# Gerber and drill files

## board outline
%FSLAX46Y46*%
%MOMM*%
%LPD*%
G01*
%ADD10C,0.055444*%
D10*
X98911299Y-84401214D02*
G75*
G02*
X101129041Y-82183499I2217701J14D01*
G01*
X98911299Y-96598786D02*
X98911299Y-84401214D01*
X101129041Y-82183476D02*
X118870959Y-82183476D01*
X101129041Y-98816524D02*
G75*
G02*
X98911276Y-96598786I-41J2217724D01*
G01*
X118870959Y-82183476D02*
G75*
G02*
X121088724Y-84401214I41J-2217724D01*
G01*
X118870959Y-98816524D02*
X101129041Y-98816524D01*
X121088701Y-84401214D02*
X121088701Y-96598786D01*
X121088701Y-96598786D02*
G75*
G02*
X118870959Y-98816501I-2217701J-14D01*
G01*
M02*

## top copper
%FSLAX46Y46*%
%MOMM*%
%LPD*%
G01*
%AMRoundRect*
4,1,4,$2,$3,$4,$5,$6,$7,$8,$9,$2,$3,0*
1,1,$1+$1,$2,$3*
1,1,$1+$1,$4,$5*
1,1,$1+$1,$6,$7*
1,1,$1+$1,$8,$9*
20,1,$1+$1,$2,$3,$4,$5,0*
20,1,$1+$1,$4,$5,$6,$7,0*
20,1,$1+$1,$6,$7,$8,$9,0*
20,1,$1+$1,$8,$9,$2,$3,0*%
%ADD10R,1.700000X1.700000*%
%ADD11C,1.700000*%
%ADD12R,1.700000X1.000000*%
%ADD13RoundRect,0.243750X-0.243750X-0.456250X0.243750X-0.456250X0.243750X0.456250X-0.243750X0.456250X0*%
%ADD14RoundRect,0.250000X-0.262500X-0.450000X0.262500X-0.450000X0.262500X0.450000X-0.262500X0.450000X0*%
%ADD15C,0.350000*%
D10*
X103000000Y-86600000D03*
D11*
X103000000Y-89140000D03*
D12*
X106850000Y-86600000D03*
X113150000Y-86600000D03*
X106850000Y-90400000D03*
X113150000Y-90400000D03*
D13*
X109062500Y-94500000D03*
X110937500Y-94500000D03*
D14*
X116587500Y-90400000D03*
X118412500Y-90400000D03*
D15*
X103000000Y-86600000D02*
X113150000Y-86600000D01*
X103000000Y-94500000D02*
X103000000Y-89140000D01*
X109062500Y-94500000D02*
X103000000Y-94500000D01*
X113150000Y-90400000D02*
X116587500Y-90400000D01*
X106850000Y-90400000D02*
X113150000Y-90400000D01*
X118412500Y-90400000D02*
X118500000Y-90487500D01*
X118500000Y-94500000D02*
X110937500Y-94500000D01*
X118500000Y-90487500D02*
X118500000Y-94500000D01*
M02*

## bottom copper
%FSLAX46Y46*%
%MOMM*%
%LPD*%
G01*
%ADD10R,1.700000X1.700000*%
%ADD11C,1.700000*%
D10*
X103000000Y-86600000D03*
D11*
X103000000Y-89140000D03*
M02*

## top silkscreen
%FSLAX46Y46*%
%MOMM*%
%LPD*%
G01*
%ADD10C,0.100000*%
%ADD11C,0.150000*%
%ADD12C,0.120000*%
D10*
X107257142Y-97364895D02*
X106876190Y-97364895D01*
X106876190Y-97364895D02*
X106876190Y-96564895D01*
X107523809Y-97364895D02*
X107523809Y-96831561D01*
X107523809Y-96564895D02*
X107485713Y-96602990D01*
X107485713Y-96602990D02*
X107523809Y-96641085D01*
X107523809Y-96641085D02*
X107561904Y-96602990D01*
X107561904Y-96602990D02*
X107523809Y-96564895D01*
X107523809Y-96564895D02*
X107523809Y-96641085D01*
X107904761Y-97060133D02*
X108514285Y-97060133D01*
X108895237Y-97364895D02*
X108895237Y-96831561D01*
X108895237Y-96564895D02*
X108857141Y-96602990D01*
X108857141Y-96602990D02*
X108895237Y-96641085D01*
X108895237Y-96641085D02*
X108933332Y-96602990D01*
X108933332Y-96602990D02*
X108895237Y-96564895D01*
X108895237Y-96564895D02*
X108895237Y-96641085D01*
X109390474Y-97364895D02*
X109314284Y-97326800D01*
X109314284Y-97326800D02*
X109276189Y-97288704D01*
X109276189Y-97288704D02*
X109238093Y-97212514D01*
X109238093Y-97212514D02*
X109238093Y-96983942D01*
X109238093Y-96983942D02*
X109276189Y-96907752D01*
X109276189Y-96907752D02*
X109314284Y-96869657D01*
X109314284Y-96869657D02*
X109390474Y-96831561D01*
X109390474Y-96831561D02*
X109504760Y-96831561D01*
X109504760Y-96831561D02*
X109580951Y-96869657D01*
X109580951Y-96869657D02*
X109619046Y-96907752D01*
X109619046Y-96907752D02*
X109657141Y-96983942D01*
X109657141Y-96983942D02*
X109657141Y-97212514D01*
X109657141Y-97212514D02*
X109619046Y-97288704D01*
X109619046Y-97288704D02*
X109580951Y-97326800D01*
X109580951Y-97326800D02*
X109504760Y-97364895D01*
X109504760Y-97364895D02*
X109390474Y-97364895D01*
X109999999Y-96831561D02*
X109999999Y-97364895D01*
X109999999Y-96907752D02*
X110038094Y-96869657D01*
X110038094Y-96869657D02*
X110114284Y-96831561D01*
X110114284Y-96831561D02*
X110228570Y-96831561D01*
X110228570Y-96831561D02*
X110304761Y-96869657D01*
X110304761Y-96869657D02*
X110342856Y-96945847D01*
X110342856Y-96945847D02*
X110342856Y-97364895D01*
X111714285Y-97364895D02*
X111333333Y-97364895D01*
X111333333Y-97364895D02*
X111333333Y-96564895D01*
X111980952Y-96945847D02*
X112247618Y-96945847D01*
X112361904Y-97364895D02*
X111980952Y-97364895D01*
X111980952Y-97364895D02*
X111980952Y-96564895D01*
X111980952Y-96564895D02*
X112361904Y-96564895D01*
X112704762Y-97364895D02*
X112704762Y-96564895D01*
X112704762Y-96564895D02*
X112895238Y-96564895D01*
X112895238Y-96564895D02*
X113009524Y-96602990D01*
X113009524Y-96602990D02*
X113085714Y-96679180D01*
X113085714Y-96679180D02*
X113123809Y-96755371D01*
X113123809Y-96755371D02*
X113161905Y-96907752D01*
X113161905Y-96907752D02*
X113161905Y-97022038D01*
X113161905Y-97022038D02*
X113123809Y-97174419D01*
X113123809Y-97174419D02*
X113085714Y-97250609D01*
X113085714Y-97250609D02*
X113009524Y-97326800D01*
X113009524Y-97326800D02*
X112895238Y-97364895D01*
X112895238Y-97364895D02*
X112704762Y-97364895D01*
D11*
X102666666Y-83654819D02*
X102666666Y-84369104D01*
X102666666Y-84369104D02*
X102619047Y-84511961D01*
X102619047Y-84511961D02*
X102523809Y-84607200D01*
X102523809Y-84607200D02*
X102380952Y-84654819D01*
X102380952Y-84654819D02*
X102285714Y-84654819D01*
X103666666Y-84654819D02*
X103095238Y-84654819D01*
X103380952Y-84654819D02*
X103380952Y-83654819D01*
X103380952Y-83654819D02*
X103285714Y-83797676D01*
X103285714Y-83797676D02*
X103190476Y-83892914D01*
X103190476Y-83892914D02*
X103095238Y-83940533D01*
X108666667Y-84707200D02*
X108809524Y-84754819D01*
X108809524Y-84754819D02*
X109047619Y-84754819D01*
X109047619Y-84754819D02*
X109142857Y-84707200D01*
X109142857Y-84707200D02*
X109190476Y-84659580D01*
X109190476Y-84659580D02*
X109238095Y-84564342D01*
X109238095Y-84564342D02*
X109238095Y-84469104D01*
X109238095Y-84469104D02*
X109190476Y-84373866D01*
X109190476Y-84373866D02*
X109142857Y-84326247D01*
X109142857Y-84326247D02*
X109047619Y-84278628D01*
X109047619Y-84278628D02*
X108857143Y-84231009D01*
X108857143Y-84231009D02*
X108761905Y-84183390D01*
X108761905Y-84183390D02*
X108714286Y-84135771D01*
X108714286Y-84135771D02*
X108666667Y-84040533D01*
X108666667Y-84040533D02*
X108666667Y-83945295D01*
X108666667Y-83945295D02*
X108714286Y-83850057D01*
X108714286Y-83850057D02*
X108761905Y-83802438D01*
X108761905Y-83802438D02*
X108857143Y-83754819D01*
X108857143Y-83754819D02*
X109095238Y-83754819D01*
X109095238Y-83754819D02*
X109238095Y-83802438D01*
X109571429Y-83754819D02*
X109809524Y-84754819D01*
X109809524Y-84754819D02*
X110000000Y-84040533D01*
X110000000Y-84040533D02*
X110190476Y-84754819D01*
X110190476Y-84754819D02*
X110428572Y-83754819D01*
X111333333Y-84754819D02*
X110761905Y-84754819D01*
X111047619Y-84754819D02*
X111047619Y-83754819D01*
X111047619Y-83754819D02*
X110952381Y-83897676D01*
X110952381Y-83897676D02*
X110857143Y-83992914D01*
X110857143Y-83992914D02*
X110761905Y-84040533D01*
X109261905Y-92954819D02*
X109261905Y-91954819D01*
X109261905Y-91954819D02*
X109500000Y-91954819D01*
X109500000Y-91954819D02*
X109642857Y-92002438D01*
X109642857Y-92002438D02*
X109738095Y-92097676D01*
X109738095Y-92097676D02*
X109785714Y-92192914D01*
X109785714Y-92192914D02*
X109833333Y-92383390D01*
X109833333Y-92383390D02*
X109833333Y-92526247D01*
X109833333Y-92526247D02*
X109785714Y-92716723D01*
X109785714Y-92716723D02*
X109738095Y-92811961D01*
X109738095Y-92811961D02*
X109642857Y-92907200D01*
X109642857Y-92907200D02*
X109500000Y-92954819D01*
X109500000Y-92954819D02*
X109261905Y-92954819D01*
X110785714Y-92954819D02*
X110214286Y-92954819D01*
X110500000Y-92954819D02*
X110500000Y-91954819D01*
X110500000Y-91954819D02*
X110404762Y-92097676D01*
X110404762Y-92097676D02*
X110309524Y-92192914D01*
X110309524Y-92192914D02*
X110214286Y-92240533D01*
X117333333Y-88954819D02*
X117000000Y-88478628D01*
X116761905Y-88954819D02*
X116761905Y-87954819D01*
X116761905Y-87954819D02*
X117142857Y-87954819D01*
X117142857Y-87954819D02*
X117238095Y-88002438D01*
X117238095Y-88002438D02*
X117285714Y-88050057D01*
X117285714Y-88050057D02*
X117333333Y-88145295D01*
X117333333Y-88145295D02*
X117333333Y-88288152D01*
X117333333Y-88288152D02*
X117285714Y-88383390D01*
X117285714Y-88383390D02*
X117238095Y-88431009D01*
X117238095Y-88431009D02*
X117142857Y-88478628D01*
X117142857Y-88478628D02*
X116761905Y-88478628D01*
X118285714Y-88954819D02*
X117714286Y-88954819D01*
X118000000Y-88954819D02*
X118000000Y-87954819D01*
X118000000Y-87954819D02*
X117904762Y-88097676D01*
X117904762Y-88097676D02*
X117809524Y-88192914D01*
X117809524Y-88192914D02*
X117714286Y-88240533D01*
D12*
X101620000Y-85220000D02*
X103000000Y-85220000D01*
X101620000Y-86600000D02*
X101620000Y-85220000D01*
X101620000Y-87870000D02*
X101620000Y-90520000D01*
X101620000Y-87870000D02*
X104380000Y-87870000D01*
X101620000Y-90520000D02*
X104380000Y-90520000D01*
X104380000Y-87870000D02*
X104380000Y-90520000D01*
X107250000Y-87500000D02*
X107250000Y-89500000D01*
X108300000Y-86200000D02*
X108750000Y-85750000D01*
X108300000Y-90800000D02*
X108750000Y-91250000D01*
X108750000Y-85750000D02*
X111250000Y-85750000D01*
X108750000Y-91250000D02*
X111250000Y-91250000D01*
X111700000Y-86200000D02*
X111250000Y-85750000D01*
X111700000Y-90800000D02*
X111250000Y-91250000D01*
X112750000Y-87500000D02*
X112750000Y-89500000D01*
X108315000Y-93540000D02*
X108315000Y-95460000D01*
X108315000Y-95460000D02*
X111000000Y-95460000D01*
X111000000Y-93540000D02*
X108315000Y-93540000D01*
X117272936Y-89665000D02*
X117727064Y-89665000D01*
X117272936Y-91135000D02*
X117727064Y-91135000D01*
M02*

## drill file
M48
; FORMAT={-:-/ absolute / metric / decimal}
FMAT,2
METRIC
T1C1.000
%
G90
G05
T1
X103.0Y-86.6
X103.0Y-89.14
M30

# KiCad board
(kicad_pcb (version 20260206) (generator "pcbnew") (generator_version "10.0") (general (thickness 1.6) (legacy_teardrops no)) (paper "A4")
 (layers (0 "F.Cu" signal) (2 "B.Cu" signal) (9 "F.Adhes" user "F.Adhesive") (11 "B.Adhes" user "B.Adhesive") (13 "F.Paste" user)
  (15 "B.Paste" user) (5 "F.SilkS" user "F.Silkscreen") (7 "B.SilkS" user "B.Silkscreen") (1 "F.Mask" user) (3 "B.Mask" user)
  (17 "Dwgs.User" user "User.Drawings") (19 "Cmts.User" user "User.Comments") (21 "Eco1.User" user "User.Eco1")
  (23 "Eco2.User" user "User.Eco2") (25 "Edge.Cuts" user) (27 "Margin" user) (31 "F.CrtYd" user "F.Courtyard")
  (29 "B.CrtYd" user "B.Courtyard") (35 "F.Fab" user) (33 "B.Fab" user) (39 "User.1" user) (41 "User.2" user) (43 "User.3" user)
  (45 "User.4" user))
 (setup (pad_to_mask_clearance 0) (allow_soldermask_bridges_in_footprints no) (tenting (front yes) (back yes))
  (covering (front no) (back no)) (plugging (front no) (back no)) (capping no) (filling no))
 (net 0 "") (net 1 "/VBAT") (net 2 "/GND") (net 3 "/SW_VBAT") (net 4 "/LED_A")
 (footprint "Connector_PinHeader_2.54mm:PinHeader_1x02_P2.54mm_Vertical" (layer "F.Cu") (at 103 86.6)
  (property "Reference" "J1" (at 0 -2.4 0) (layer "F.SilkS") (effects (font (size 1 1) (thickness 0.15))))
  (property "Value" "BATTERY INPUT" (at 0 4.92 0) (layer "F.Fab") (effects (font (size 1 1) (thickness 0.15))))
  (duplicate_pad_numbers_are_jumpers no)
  (fp_line (start -1.38 -1.38) (end 0 -1.38) (stroke (width 0.12) (type solid)) (layer "F.SilkS"))
  (fp_line (start -1.38 0) (end -1.38 -1.38) (stroke (width 0.12) (type solid)) (layer "F.SilkS"))
  (fp_line (start -1.38 1.27) (end -1.38 3.92) (stroke (width 0.12) (type solid)) (layer "F.SilkS"))
  (fp_line (start -1.38 1.27) (end 1.38 1.27) (stroke (width 0.12) (type solid)) (layer "F.SilkS"))
  (fp_line (start -1.38 3.92) (end 1.38 3.92) (stroke (width 0.12) (type solid)) (layer "F.SilkS"))
  (fp_line (start 1.38 1.27) (end 1.38 3.92) (stroke (width 0.12) (type solid)) (layer "F.SilkS"))
  (pad "1" thru_hole rect (at 0 0) (size 1.7 1.7) (drill 1) (layers "*.Cu" "*.Mask") (remove_unused_layers no) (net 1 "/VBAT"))
  (pad "2" thru_hole circle (at 0 2.54) (size 1.7 1.7) (drill 1) (layers "*.Cu" "*.Mask") (remove_unused_layers no) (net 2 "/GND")))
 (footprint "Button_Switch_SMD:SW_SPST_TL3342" (layer "F.Cu") (at 110 88.5)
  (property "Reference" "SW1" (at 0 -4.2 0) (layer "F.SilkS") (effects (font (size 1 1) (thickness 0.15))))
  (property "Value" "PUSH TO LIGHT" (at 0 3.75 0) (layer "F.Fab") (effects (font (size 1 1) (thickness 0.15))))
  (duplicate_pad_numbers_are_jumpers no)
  (fp_line (start -2.75 -1) (end -2.75 1) (stroke (width 0.12) (type solid)) (layer "F.SilkS"))
  (fp_line (start -1.7 -2.3) (end -1.25 -2.75) (stroke (width 0.12) (type solid)) (layer "F.SilkS"))
  (fp_line (start -1.7 2.3) (end -1.25 2.75) (stroke (width 0.12) (type solid)) (layer "F.SilkS"))
  (fp_line (start -1.25 -2.75) (end 1.25 -2.75) (stroke (width 0.12) (type solid)) (layer "F.SilkS"))
  (fp_line (start -1.25 2.75) (end 1.25 2.75) (stroke (width 0.12) (type solid)) (layer "F.SilkS"))
  (fp_line (start 1.7 -2.3) (end 1.25 -2.75) (stroke (width 0.12) (type solid)) (layer "F.SilkS"))
  (fp_line (start 1.7 2.3) (end 1.25 2.75) (stroke (width 0.12) (type solid)) (layer "F.SilkS"))
  (fp_line (start 2.75 -1) (end 2.75 1) (stroke (width 0.12) (type solid)) (layer "F.SilkS"))
  (pad "1" smd rect (at -3.15 -1.9) (size 1.7 1) (layers "F.Cu" "F.Mask" "F.Paste") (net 1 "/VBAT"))
  (pad "1" smd rect (at 3.15 -1.9) (size 1.7 1) (layers "F.Cu" "F.Mask" "F.Paste") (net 1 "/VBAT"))
  (pad "2" smd rect (at -3.15 1.9) (size 1.7 1) (layers "F.Cu" "F.Mask" "F.Paste") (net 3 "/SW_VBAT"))
  (pad "2" smd rect (at 3.15 1.9) (size 1.7 1) (layers "F.Cu" "F.Mask" "F.Paste") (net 3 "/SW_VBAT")))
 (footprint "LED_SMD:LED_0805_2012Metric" (layer "F.Cu") (at 110 94.5)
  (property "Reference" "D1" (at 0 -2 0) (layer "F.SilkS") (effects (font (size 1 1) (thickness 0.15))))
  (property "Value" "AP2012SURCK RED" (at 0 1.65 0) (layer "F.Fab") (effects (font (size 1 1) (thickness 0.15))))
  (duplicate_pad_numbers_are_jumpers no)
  (fp_line (start -1.685 -0.96) (end -1.685 0.96) (stroke (width 0.12) (type solid)) (layer "F.SilkS"))
  (fp_line (start -1.685 0.96) (end 1 0.96) (stroke (width 0.12) (type solid)) (layer "F.SilkS"))
  (fp_line (start 1 -0.96) (end -1.685 -0.96) (stroke (width 0.12) (type solid)) (layer "F.SilkS"))
  (pad "1" smd roundrect (at -0.9375 0) (size 0.975 1.4) (layers "F.Cu" "F.Mask" "F.Paste") (roundrect_rratio 0.25) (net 2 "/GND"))
  (pad "2" smd roundrect (at 0.9375 0) (size 0.975 1.4) (layers "F.Cu" "F.Mask" "F.Paste") (roundrect_rratio 0.25) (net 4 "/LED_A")))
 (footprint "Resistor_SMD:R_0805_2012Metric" (layer "F.Cu") (at 117.5 90.4)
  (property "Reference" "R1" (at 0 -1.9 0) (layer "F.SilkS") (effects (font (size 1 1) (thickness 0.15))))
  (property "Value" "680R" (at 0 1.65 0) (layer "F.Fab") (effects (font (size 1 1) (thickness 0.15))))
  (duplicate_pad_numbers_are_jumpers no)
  (fp_line (start -0.227064 -0.735) (end 0.227064 -0.735) (stroke (width 0.12) (type solid)) (layer "F.SilkS"))
  (fp_line (start -0.227064 0.735) (end 0.227064 0.735) (stroke (width 0.12) (type solid)) (layer "F.SilkS"))
  (pad "1" smd roundrect (at -0.9125 0) (size 1.025 1.4) (layers "F.Cu" "F.Mask" "F.Paste") (roundrect_rratio 0.243902) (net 3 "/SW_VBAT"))
  (pad "2" smd roundrect (at 0.9125 0) (size 1.025 1.4) (layers "F.Cu" "F.Mask" "F.Paste") (roundrect_rratio 0.243902) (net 4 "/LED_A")))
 (gr_arc (start 98.911299 84.401214) (mid 99.560861 82.833034) (end 101.129041 82.183476) (stroke (width 0.055444) (type default))
  (layer "Edge.Cuts"))
 (gr_line (start 98.911299 96.598786) (end 98.911299 84.401214) (stroke (width 0.055444) (type default)) (layer "Edge.Cuts"))
 (gr_line (start 101.129041 82.183476) (end 118.870959 82.183476) (stroke (width 0.055444) (type default)) (layer "Edge.Cuts"))
 (gr_arc (start 101.129041 98.816524) (mid 99.560863 98.166964) (end 98.911299 96.598786) (stroke (width 0.055444) (type default))
  (layer "Edge.Cuts"))
 (gr_arc (start 118.870959 82.183476) (mid 120.439137 82.833036) (end 121.088701 84.401214) (stroke (width 0.055444) (type default))
  (layer "Edge.Cuts"))
 (gr_line (start 118.870959 98.816524) (end 101.129041 98.816524) (stroke (width 0.055444) (type default)) (layer "Edge.Cuts"))
 (gr_line (start 121.088701 84.401214) (end 121.088701 96.598786) (stroke (width 0.055444) (type default)) (layer "Edge.Cuts"))
 (gr_arc (start 121.088701 96.598786) (mid 120.439139 98.166966) (end 118.870959 98.816524) (stroke (width 0.055444) (type default))
  (layer "Edge.Cuts"))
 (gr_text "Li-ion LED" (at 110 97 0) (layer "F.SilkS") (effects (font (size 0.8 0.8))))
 (segment (start 103 86.6) (end 113.15 86.6) (width 0.35) (layer "F.Cu") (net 1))
 (segment (start 103 94.5) (end 103 89.14) (width 0.35) (layer "F.Cu") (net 2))
 (segment (start 109.0625 94.5) (end 103 94.5) (width 0.35) (layer "F.Cu") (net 2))
 (segment (start 113.15 90.4) (end 116.5875 90.4) (width 0.35) (layer "F.Cu") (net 3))
 (segment (start 106.85 90.4) (end 113.15 90.4) (width 0.35) (layer "F.Cu") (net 3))
 (segment (start 118.4125 90.4) (end 118.5 90.4875) (width 0.35) (layer "F.Cu") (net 4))
 (segment (start 118.5 94.5) (end 110.9375 94.5) (width 0.35) (layer "F.Cu") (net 4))
 (segment (start 118.5 90.4875) (end 118.5 94.5) (width 0.35) (layer "F.Cu") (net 4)))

